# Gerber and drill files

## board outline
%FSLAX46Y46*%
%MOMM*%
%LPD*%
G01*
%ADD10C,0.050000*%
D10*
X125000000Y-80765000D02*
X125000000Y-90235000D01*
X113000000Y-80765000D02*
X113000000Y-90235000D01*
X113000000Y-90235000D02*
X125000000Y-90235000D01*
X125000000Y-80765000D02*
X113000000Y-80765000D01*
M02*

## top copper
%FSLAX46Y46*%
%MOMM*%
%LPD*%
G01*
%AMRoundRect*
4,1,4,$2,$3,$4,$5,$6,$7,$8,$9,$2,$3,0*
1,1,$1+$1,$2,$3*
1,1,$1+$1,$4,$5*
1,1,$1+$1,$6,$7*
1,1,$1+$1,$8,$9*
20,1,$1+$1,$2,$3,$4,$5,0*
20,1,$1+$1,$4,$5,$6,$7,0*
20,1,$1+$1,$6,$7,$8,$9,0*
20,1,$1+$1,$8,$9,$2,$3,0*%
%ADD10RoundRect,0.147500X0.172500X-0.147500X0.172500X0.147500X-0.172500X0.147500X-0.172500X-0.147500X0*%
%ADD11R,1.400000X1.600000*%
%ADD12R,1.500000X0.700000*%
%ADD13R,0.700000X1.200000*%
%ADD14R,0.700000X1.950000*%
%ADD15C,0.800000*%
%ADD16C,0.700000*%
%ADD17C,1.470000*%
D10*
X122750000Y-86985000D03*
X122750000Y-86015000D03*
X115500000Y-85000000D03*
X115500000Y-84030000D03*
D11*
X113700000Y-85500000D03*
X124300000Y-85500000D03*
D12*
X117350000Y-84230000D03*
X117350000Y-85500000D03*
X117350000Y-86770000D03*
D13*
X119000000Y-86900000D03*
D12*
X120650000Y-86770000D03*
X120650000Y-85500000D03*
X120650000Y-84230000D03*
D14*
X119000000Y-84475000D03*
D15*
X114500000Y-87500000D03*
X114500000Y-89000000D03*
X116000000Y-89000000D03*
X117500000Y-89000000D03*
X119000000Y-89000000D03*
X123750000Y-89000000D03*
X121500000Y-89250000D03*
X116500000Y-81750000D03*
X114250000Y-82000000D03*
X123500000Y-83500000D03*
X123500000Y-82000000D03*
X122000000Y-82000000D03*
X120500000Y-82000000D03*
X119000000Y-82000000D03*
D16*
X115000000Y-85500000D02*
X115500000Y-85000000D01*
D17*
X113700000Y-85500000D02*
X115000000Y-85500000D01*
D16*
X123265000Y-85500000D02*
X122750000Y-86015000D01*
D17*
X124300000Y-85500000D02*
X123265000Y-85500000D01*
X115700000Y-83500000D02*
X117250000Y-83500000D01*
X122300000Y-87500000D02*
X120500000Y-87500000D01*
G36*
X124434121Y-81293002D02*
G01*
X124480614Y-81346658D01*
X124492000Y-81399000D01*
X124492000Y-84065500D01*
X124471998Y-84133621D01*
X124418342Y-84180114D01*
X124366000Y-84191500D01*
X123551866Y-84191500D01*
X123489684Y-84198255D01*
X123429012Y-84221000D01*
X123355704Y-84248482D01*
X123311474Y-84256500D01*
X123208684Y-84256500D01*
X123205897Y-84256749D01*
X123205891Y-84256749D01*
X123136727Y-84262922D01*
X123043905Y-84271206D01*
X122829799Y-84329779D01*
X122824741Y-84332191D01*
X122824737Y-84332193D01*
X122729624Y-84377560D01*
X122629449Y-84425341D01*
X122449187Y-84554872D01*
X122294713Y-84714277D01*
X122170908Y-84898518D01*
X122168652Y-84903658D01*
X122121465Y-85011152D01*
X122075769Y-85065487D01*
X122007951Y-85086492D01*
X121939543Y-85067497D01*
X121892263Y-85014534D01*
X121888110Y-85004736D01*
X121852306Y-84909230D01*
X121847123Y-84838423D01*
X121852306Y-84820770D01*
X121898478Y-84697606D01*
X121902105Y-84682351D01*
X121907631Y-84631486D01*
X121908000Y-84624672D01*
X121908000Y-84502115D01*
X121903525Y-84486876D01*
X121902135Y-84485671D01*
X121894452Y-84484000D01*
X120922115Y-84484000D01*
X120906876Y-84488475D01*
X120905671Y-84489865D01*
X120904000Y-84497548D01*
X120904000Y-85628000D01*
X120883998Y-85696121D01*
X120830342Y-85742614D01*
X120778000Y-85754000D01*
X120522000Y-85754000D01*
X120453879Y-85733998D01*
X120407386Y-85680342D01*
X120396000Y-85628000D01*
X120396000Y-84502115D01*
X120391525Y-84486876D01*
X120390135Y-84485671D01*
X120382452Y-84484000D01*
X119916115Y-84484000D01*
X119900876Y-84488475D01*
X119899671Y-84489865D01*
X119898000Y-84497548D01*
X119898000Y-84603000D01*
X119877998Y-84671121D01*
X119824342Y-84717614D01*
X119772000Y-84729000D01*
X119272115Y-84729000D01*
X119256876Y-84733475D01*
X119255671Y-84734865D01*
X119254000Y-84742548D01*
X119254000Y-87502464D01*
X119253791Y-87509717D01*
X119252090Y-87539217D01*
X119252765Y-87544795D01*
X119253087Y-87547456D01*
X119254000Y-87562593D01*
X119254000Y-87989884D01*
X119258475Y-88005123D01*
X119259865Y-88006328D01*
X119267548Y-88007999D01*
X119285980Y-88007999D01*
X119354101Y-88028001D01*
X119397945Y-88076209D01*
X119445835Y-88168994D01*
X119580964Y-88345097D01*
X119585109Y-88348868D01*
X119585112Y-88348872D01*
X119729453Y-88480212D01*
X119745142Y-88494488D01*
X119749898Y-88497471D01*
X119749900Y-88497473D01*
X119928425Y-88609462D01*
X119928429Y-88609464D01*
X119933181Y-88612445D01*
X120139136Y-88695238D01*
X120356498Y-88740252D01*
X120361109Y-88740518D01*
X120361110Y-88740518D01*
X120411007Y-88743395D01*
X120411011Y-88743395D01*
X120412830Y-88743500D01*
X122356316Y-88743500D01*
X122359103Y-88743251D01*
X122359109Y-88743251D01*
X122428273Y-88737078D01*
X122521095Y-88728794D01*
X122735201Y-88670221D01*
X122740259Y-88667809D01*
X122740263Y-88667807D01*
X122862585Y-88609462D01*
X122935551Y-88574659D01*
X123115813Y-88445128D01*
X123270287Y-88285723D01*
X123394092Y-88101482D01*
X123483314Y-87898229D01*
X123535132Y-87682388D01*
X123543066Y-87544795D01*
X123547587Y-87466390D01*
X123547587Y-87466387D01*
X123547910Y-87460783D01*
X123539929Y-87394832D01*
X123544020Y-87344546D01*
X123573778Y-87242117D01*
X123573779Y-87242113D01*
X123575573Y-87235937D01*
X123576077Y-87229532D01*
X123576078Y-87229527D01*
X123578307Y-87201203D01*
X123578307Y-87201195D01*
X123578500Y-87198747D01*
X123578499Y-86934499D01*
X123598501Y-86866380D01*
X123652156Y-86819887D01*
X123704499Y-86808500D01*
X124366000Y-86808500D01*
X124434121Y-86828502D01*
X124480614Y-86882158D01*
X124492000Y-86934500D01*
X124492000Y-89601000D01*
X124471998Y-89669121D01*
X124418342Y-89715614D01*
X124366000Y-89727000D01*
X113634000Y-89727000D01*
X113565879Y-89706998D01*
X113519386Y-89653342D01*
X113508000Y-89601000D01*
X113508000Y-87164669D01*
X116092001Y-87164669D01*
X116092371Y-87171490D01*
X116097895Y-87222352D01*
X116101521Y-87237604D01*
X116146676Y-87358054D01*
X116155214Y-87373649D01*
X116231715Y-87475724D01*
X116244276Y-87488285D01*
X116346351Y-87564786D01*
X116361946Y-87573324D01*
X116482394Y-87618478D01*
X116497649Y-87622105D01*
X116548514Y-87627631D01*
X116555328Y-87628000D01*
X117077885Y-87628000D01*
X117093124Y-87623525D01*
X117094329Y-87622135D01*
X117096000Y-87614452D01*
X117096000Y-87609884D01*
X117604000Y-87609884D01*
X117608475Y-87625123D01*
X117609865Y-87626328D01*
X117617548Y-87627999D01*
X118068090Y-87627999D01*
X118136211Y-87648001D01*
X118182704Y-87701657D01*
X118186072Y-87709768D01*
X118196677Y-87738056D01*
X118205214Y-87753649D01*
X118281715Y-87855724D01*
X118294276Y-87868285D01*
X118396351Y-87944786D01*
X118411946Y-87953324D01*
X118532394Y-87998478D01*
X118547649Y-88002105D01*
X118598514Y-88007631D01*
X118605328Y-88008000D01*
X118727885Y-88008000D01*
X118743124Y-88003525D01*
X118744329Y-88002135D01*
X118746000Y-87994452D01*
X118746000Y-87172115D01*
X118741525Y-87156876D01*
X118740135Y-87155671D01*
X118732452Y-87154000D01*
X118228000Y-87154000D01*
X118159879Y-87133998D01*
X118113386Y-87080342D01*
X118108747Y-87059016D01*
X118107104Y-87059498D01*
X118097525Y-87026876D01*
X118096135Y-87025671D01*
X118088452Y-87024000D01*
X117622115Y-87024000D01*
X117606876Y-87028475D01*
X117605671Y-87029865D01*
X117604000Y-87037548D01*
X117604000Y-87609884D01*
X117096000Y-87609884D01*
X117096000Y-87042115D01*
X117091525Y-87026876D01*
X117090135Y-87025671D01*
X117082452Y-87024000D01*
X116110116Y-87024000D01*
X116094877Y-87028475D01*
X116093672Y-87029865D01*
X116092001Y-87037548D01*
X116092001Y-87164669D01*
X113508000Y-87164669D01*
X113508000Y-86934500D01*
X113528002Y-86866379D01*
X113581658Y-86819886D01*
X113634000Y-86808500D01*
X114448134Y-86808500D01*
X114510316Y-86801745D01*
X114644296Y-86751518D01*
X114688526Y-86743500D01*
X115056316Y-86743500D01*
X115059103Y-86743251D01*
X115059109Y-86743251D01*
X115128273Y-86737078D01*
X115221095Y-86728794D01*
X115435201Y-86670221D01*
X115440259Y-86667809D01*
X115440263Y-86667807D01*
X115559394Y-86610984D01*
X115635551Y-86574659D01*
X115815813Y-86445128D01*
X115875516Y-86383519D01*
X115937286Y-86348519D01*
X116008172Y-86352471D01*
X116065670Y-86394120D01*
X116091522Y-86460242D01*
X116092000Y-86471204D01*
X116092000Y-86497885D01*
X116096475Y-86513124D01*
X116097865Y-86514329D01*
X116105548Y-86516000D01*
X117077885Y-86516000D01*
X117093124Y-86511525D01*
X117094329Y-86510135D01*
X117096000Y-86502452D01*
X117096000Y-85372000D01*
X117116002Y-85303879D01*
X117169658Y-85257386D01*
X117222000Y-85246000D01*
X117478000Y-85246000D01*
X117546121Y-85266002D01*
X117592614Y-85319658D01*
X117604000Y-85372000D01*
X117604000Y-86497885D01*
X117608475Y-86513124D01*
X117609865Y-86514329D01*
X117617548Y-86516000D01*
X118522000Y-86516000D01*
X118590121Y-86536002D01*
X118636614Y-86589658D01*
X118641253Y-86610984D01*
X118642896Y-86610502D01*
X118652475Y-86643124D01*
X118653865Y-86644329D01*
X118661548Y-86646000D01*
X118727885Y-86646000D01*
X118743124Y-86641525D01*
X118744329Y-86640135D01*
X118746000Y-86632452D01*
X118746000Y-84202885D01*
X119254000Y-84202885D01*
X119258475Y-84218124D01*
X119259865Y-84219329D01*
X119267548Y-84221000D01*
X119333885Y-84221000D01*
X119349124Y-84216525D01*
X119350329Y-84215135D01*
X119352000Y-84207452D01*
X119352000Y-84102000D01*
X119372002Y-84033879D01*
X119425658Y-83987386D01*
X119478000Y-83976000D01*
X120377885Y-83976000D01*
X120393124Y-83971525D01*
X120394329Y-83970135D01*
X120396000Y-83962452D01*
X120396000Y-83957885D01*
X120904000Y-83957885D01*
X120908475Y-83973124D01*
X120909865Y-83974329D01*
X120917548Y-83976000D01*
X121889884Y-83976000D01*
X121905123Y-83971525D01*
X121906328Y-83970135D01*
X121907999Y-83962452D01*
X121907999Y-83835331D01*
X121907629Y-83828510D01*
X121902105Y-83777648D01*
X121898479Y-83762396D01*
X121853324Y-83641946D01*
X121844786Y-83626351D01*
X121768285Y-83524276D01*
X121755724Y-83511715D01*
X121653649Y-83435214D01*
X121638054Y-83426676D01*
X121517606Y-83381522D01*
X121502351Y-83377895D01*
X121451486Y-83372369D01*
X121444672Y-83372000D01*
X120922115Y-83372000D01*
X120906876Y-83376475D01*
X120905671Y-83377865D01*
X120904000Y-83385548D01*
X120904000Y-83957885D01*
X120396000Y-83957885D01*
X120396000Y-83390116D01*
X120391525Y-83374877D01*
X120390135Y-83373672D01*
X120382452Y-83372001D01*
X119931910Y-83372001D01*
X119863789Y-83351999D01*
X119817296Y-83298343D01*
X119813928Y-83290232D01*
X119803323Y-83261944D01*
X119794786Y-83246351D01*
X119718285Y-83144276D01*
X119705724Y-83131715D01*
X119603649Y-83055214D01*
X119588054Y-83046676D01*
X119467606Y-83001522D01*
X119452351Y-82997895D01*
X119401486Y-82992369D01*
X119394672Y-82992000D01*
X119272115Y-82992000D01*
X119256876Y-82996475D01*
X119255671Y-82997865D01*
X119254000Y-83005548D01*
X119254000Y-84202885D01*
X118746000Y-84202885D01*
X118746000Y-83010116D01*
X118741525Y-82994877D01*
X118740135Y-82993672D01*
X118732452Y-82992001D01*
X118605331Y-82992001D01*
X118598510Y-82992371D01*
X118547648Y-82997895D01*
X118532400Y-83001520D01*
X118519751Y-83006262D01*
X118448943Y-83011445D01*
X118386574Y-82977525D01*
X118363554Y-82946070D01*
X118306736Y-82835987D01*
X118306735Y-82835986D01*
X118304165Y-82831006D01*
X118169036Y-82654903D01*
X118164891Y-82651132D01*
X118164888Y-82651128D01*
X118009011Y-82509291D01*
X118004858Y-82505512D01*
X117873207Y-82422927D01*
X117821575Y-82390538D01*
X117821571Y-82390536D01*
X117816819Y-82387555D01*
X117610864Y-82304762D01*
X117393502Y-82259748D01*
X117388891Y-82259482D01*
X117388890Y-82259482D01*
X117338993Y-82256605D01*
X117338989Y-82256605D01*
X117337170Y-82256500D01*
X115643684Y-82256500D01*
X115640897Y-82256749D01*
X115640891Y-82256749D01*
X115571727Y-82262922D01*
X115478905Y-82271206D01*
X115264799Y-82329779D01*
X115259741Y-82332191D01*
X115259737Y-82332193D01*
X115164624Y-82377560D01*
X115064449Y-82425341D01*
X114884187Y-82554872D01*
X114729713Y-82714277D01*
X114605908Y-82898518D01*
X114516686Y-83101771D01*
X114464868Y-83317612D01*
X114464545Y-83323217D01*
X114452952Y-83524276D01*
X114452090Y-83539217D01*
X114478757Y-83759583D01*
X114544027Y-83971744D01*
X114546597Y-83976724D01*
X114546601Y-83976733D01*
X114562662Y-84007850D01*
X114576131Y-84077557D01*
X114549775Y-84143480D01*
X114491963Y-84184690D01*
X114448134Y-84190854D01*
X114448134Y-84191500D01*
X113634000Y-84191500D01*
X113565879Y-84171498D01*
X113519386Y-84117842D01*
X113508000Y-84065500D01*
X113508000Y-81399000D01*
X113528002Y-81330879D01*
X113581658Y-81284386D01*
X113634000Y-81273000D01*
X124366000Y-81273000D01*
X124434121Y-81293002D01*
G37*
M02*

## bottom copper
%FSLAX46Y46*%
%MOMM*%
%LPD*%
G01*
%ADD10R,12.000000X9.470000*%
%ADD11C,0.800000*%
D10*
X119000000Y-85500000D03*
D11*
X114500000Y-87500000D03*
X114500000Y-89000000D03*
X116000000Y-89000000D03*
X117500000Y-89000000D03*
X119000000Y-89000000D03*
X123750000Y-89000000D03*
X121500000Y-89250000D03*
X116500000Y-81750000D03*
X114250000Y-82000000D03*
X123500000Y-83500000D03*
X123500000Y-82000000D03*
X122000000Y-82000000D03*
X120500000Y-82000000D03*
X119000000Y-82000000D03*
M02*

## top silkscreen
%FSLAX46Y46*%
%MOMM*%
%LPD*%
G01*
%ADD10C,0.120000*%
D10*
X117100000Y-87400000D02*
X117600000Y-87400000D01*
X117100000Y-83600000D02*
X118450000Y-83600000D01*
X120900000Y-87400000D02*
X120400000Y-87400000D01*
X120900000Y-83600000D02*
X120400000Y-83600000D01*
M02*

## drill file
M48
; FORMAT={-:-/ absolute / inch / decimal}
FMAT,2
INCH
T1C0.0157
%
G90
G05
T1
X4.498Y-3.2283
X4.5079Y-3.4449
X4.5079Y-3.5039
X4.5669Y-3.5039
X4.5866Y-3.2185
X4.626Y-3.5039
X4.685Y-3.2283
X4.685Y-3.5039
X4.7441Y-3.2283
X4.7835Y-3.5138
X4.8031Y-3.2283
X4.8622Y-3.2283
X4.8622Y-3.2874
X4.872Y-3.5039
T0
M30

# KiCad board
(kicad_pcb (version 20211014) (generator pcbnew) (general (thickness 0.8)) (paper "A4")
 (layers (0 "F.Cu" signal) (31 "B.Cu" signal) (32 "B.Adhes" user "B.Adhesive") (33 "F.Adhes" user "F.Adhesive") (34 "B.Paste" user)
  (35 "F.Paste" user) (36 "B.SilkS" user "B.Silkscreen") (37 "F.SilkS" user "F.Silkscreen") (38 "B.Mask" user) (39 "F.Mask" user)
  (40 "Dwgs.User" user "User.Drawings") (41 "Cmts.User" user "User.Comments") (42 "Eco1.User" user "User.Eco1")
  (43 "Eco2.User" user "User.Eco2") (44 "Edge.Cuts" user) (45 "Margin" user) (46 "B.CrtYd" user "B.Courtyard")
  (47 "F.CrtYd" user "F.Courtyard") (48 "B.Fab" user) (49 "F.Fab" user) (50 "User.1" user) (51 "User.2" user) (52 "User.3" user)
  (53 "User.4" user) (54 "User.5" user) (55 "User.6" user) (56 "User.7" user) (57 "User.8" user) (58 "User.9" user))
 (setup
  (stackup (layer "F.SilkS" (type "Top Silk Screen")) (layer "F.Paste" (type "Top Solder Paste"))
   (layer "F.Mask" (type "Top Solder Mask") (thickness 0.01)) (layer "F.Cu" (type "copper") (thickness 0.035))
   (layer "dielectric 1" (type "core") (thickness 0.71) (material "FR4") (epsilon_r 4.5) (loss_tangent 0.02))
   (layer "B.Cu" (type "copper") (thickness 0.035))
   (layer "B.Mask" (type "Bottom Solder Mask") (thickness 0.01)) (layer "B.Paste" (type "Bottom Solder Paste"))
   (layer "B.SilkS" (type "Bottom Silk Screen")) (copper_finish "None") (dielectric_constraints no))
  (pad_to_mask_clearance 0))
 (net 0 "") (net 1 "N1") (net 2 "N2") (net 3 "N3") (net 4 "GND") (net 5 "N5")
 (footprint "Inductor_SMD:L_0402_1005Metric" (layer "F.Cu") (at 115.5 84.515 90)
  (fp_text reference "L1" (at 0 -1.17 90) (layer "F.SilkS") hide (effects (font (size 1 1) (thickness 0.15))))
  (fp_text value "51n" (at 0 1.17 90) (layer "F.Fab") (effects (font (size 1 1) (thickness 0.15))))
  (pad "1" smd roundrect (at -0.485 0 90) (size 0.59 0.64) (layers "F.Cu" "F.Paste" "F.Mask") (roundrect_rratio 0.25) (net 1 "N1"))
  (pad "2" smd roundrect (at 0.485 0 90) (size 0.59 0.64) (layers "F.Cu" "F.Paste" "F.Mask") (roundrect_rratio 0.25) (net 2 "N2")))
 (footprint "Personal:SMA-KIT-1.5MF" (layer "F.Cu") (at 119 85.5)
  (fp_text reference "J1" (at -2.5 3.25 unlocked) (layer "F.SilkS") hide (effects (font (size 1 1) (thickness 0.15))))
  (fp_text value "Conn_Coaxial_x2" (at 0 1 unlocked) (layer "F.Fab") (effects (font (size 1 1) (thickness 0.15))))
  (fp_line (start -6 -4.735) (end -6 4.735) (layer "Edge.Cuts") (width 0.05))
  (fp_line (start -6 4.735) (end 6 4.735) (layer "Edge.Cuts") (width 0.05))
  (fp_line (start 6 -4.735) (end -6 -4.735) (layer "Edge.Cuts") (width 0.05))
  (fp_line (start 6 -4.735) (end 6 4.735) (layer "Edge.Cuts") (width 0.05))
  (pad "1" smd rect (at -5.3 0) (size 1.4 1.6) (layers "F.Cu" "F.Paste" "F.Mask") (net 1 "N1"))
  (pad "2" smd rect (at 5.3 0) (size 1.4 1.6) (layers "F.Cu" "F.Paste" "F.Mask") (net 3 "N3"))
  (pad "3" smd rect (at 0 0) (size 12 9.47) (layers "B.Cu" "B.Paste" "B.Mask") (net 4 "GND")))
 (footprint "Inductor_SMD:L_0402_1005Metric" (layer "F.Cu") (at 122.75 86.5 90)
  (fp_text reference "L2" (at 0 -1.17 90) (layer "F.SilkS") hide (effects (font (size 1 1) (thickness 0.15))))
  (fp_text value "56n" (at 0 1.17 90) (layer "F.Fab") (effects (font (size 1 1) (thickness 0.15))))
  (pad "1" smd roundrect (at -0.485 0 90) (size 0.59 0.64) (layers "F.Cu" "F.Paste" "F.Mask") (roundrect_rratio 0.25) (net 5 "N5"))
  (pad "2" smd roundrect (at 0.485 0 90) (size 0.59 0.64) (layers "F.Cu" "F.Paste" "F.Mask") (roundrect_rratio 0.25) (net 3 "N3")))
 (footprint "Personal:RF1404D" (layer "F.Cu") (at 119 85.5)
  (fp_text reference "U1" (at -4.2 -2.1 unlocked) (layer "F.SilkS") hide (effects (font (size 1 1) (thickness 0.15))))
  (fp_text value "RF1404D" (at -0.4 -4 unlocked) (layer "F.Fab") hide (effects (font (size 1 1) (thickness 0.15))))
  (fp_line (start 1.9 -1.9) (end 1.4 -1.9) (layer "F.SilkS") (width 0.12))
  (fp_line (start 1.9 1.9) (end 1.4 1.9) (layer "F.SilkS") (width 0.12))
  (fp_line (start -1.9 -1.9) (end -0.55 -1.9) (layer "F.SilkS") (width 0.12))
  (fp_line (start -1.9 1.9) (end -1.4 1.9) (layer "F.SilkS") (width 0.12))
  (pad "1" smd rect (at -1.65 -1.27 90) (size 0.7 1.5) (layers "F.Cu" "F.Paste" "F.Mask") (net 2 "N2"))
  (pad "2" smd rect (at -1.65 0 90) (size 0.7 1.5) (layers "F.Cu" "F.Paste" "F.Mask") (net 4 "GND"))
  (pad "3" smd rect (at -1.65 1.27 90) (size 0.7 1.5) (layers "F.Cu" "F.Paste" "F.Mask") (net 4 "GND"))
  (pad "4" smd rect (at 0 1.4) (size 0.7 1.2) (layers "F.Cu" "F.Paste" "F.Mask") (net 4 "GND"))
  (pad "5" smd rect (at 1.65 1.27 270) (size 0.7 1.5) (layers "F.Cu" "F.Paste" "F.Mask") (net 5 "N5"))
  (pad "6" smd rect (at 1.65 0 270) (size 0.7 1.5) (layers "F.Cu" "F.Paste" "F.Mask") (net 4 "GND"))
  (pad "7" smd rect (at 1.65 -1.27 270) (size 0.7 1.5) (layers "F.Cu" "F.Paste" "F.Mask") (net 4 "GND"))
  (pad "8" smd rect (at 0 -1.025 180) (size 0.7 1.95) (layers "F.Cu" "F.Paste" "F.Mask") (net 4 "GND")))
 (segment (start 115 85.5) (end 115.5 85) (width 0.7) (layer "F.Cu") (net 1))
 (segment (start 113.7 85.5) (end 115 85.5) (width 1.47) (layer "F.Cu") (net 1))
 (via (at 117.5 89) (size 0.8) (drill 0.4) (layers "F.Cu" "B.Cu") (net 4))
 (via (at 114.5 87.5) (size 0.8) (drill 0.4) (layers "F.Cu" "B.Cu") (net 4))
 (via (at 119 89) (size 0.8) (drill 0.4) (layers "F.Cu" "B.Cu") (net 4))
 (via (at 119 82) (size 0.8) (drill 0.4) (layers "F.Cu" "B.Cu") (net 4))
 (via (at 123.75 89) (size 0.8) (drill 0.4) (layers "F.Cu" "B.Cu") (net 4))
 (via (at 116.5 81.75) (size 0.8) (drill 0.4) (layers "F.Cu" "B.Cu") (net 4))
 (via (at 123.5 83.5) (size 0.8) (drill 0.4) (layers "F.Cu" "B.Cu") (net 4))
 (via (at 114.5 89) (size 0.8) (drill 0.4) (layers "F.Cu" "B.Cu") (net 4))
 (via (at 120.5 82) (size 0.8) (drill 0.4) (layers "F.Cu" "B.Cu") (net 4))
 (via (at 116 89) (size 0.8) (drill 0.4) (layers "F.Cu" "B.Cu") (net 4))
 (via (at 122 82) (size 0.8) (drill 0.4) (layers "F.Cu" "B.Cu") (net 4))
 (via (at 121.5 89.25) (size 0.8) (drill 0.4) (layers "F.Cu" "B.Cu") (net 4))
 (via (at 123.5 82) (size 0.8) (drill 0.4) (layers "F.Cu" "B.Cu") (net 4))
 (via (at 114.25 82) (size 0.8) (drill 0.4) (layers "F.Cu" "B.Cu") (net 4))
 (segment (start 123.265 85.5) (end 122.75 86.015) (width 0.7) (layer "F.Cu") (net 3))
 (segment (start 124.3 85.5) (end 123.265 85.5) (width 1.47) (layer "F.Cu") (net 3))
 (segment (start 115.7 83.5) (end 117.25 83.5) (width 1.47) (layer "F.Cu") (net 2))
 (segment (start 122.3 87.5) (end 120.5 87.5) (width 1.47) (layer "F.Cu") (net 5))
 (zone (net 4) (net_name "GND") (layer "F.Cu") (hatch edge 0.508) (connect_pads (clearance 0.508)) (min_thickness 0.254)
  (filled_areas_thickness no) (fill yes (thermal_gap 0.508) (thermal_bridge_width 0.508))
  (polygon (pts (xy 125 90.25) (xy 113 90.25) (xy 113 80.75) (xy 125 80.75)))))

